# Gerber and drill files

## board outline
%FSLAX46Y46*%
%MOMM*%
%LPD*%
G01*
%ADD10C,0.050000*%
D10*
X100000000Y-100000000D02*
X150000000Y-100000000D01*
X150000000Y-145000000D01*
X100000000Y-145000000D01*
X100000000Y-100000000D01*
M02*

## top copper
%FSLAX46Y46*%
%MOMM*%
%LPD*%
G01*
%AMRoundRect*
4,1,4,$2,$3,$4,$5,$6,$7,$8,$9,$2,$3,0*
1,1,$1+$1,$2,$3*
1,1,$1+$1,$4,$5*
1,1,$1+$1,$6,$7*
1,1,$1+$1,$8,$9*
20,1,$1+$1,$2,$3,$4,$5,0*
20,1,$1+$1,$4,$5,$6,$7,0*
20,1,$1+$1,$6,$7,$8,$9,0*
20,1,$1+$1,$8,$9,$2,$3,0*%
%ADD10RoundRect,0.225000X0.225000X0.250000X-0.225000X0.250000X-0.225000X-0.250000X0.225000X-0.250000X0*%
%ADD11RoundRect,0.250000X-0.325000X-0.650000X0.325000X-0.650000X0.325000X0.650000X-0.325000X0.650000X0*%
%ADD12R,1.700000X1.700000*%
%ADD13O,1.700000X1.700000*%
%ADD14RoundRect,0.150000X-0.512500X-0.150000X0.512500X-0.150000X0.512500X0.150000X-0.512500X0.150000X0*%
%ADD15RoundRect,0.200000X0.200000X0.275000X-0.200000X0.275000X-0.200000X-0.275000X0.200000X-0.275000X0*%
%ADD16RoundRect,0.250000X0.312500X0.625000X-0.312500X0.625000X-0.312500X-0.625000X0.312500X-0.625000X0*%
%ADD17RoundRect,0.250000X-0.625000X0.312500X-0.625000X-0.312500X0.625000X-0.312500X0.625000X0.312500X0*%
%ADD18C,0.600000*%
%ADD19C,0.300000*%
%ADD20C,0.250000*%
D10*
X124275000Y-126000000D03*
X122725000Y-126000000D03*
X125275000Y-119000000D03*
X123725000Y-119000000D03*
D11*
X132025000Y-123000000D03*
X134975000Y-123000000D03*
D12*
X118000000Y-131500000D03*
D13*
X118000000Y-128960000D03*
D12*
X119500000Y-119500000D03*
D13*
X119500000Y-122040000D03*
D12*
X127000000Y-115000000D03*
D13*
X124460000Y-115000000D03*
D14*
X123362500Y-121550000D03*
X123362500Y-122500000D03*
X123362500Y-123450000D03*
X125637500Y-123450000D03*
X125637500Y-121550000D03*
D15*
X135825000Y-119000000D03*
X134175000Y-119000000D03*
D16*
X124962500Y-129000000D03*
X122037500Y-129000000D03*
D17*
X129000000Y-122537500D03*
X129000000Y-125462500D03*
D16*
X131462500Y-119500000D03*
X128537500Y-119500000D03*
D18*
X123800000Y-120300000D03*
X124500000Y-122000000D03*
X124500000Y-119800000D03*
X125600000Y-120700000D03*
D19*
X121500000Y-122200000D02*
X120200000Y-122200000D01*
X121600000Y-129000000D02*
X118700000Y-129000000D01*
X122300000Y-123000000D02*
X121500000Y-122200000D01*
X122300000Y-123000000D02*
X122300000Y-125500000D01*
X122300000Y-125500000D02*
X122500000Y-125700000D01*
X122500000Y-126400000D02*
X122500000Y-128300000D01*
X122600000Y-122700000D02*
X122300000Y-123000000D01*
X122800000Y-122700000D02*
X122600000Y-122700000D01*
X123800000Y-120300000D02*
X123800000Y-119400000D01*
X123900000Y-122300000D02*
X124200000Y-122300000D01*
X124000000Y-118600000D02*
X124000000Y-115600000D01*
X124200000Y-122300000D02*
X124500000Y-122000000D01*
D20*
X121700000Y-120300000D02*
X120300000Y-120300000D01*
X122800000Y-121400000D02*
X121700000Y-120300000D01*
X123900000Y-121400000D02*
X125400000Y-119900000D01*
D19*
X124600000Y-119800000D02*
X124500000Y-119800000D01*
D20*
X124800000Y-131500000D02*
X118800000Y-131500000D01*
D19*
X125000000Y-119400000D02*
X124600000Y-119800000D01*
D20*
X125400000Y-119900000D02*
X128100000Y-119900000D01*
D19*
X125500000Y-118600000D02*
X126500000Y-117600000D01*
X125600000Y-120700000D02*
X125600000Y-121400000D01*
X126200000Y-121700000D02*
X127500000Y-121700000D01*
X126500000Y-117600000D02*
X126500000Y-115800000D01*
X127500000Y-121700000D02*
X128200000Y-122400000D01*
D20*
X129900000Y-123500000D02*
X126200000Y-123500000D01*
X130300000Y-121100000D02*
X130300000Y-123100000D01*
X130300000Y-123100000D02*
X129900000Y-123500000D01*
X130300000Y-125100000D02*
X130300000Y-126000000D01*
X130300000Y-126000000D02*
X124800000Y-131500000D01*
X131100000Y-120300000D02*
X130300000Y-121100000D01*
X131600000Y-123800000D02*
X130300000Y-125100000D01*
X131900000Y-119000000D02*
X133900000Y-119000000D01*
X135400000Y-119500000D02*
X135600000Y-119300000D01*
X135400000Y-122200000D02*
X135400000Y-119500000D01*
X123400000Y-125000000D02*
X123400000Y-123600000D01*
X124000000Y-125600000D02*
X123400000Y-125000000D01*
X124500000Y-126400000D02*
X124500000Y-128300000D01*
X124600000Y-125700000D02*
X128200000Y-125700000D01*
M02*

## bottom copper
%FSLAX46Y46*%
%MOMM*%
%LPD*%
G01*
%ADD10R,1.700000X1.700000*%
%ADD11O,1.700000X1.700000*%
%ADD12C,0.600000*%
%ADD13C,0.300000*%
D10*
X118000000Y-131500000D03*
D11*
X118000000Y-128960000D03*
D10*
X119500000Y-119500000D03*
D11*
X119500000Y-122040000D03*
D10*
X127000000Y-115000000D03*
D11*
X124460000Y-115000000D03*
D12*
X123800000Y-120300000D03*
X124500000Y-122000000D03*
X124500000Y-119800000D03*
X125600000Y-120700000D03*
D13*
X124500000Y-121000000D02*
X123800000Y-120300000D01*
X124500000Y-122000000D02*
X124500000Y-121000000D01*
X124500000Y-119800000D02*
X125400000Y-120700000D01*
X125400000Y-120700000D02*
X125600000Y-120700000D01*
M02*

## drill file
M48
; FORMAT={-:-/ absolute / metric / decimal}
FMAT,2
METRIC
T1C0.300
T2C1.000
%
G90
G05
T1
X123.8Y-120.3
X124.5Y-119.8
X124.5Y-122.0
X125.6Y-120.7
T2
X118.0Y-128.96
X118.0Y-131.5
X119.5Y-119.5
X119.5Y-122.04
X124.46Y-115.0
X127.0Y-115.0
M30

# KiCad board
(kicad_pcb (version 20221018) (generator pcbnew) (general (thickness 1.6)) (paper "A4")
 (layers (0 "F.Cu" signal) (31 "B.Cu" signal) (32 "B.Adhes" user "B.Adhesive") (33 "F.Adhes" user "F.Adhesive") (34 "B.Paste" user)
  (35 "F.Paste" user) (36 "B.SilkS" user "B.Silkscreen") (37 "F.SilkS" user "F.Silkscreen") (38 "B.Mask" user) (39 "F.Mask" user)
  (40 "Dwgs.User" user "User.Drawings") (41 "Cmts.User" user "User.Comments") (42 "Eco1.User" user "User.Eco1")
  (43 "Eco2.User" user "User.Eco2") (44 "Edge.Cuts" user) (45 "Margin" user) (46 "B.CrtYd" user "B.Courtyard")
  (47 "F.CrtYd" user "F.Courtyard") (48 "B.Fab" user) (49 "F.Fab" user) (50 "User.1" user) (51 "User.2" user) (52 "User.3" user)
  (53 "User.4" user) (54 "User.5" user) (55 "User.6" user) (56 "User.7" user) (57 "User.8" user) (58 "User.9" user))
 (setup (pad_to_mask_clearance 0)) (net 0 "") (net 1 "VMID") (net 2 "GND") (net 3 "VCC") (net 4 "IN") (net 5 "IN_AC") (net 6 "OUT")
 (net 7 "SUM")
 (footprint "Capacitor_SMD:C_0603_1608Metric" (layer "F.Cu") (at 123.5 126 180)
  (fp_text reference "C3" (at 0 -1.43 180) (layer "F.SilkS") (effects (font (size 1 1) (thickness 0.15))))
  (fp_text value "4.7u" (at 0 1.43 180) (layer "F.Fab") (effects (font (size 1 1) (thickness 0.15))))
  (pad "1" smd roundrect (at -0.775 0 180) (size 0.9 0.95) (layers "F.Cu" "F.Paste" "F.Mask") (roundrect_rratio 0.25) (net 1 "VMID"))
  (pad "2" smd roundrect (at 0.775 0 180) (size 0.9 0.95) (layers "F.Cu" "F.Paste" "F.Mask") (roundrect_rratio 0.25) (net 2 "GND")))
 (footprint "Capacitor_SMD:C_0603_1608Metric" (layer "F.Cu") (at 124.5 119 180)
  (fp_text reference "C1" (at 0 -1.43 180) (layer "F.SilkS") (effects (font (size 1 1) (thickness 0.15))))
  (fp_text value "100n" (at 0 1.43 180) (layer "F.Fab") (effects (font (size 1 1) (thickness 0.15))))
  (pad "1" smd roundrect (at -0.775 0 180) (size 0.9 0.95) (layers "F.Cu" "F.Paste" "F.Mask") (roundrect_rratio 0.25) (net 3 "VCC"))
  (pad "2" smd roundrect (at 0.775 0 180) (size 0.9 0.95) (layers "F.Cu" "F.Paste" "F.Mask") (roundrect_rratio 0.25) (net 2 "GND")))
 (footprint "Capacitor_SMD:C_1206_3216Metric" (layer "F.Cu") (at 133.5 123)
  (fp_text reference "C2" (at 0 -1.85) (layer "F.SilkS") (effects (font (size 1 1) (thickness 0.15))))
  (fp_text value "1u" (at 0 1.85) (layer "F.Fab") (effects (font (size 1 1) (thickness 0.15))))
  (pad "1" smd roundrect (at -1.475 0) (size 1.15 1.8) (layers "F.Cu" "F.Paste" "F.Mask") (roundrect_rratio 0.217391) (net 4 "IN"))
  (pad "2" smd roundrect (at 1.475 0) (size 1.15 1.8) (layers "F.Cu" "F.Paste" "F.Mask") (roundrect_rratio 0.217391) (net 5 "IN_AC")))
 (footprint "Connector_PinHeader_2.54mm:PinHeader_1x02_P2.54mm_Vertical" (layer "F.Cu") (at 118 131.5 180)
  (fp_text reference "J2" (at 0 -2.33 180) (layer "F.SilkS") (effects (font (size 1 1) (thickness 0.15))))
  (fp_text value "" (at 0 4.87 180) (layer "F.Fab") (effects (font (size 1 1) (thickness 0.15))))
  (pad "1" thru_hole rect (at 0 0 180) (size 1.7 1.7) (drill 1) (layers "*.Cu" "*.Mask") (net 4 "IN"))
  (pad "2" thru_hole oval (at 0 2.54 180) (size 1.7 1.7) (drill 1) (layers "*.Cu" "*.Mask") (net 2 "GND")))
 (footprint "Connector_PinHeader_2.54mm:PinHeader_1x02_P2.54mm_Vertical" (layer "F.Cu") (at 119.5 119.5)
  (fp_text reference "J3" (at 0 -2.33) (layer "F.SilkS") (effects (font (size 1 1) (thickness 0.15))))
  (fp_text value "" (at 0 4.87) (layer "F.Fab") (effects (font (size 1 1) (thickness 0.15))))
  (pad "1" thru_hole rect (at 0 0) (size 1.7 1.7) (drill 1) (layers "*.Cu" "*.Mask") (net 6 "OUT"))
  (pad "2" thru_hole oval (at 0 2.54) (size 1.7 1.7) (drill 1) (layers "*.Cu" "*.Mask") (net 2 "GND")))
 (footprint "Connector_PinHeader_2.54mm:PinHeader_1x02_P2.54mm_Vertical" (layer "F.Cu") (at 127 115 -90)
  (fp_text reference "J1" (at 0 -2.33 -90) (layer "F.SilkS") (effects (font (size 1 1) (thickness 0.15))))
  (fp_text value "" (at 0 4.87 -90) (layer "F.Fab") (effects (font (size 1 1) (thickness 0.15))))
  (pad "1" thru_hole rect (at 0 0 270) (size 1.7 1.7) (drill 1) (layers "*.Cu" "*.Mask") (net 3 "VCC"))
  (pad "2" thru_hole oval (at 0 2.54 270) (size 1.7 1.7) (drill 1) (layers "*.Cu" "*.Mask") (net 2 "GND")))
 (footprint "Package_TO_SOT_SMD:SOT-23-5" (layer "F.Cu") (at 124.5 122.5)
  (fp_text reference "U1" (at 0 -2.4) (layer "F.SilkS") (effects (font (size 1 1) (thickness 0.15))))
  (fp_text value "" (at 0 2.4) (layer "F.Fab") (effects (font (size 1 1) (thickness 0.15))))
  (pad "1" smd roundrect (at -1.1375 -0.95) (size 1.325 0.6) (layers "F.Cu" "F.Paste" "F.Mask") (roundrect_rratio 0.25) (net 6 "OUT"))
  (pad "2" smd roundrect (at -1.1375 0) (size 1.325 0.6) (layers "F.Cu" "F.Paste" "F.Mask") (roundrect_rratio 0.25) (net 2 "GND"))
  (pad "3" smd roundrect (at -1.1375 0.95) (size 1.325 0.6) (layers "F.Cu" "F.Paste" "F.Mask") (roundrect_rratio 0.25) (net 1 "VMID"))
  (pad "4" smd roundrect (at 1.1375 0.95) (size 1.325 0.6) (layers "F.Cu" "F.Paste" "F.Mask") (roundrect_rratio 0.25) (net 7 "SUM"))
  (pad "5" smd roundrect (at 1.1375 -0.95) (size 1.325 0.6) (layers "F.Cu" "F.Paste" "F.Mask") (roundrect_rratio 0.25) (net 3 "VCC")))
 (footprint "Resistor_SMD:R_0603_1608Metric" (layer "F.Cu") (at 135 119 180)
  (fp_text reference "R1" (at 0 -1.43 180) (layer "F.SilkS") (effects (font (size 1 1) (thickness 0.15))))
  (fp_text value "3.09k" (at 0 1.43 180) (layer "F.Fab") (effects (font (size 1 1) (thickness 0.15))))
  (pad "1" smd roundrect (at -0.825 0 180) (size 0.8 0.95) (layers "F.Cu" "F.Paste" "F.Mask") (roundrect_rratio 0.25) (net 5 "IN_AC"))
  (pad "2" smd roundrect (at 0.825 0 180) (size 0.8 0.95) (layers "F.Cu" "F.Paste" "F.Mask") (roundrect_rratio 0.25) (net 7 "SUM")))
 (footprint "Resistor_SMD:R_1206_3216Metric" (layer "F.Cu") (at 123.5 129 180)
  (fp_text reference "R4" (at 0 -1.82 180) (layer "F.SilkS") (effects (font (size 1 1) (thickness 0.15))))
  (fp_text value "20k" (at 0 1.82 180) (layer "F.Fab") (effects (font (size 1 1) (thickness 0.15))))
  (pad "1" smd roundrect (at -1.4625 0 180) (size 1.125 1.75) (layers "F.Cu" "F.Paste" "F.Mask") (roundrect_rratio 0.222222) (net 1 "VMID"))
  (pad "2" smd roundrect (at 1.4625 0 180) (size 1.125 1.75) (layers "F.Cu" "F.Paste" "F.Mask") (roundrect_rratio 0.222222) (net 2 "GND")))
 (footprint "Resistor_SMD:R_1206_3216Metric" (layer "F.Cu") (at 129 124 -90)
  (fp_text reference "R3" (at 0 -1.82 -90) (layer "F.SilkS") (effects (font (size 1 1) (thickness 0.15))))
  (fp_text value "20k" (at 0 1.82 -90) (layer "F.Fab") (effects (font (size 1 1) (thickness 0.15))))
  (pad "1" smd roundrect (at -1.4625 0 270) (size 1.125 1.75) (layers "F.Cu" "F.Paste" "F.Mask") (roundrect_rratio 0.222222) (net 3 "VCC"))
  (pad "2" smd roundrect (at 1.4625 0 270) (size 1.125 1.75) (layers "F.Cu" "F.Paste" "F.Mask") (roundrect_rratio 0.222222) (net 1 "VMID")))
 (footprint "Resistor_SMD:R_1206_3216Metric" (layer "F.Cu") (at 130 119.5 180)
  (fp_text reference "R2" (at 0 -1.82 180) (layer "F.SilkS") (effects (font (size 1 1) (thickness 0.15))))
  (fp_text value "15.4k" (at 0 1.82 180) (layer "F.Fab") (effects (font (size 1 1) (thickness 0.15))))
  (pad "1" smd roundrect (at -1.4625 0 180) (size 1.125 1.75) (layers "F.Cu" "F.Paste" "F.Mask") (roundrect_rratio 0.222222) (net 7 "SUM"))
  (pad "2" smd roundrect (at 1.4625 0 180) (size 1.125 1.75) (layers "F.Cu" "F.Paste" "F.Mask") (roundrect_rratio 0.222222) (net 6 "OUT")))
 (gr_rect (start 100 100) (end 150 145) (stroke (width 0.05) (type default)) (fill none) (layer "Edge.Cuts"))
 (segment (start 121.5 122.2) (end 120.2 122.2) (width 0.3) (layer "F.Cu") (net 2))
 (segment (start 121.6 129) (end 118.7 129) (width 0.3) (layer "F.Cu") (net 2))
 (segment (start 122.3 123) (end 121.5 122.2) (width 0.3) (layer "F.Cu") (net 2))
 (segment (start 122.3 123) (end 122.3 125.5) (width 0.3) (layer "F.Cu") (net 2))
 (segment (start 122.3 125.5) (end 122.5 125.7) (width 0.3) (layer "F.Cu") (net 2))
 (segment (start 122.5 126.4) (end 122.5 128.3) (width 0.3) (layer "F.Cu") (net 2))
 (segment (start 122.6 122.7) (end 122.3 123) (width 0.3) (layer "F.Cu") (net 2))
 (segment (start 122.8 122.7) (end 122.6 122.7) (width 0.3) (layer "F.Cu") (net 2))
 (segment (start 123.8 120.3) (end 123.8 119.4) (width 0.3) (layer "F.Cu") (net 2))
 (segment (start 123.9 122.3) (end 124.2 122.3) (width 0.3) (layer "F.Cu") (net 2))
 (segment (start 124 118.6) (end 124 115.6) (width 0.3) (layer "F.Cu") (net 2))
 (segment (start 124.2 122.3) (end 124.5 122) (width 0.3) (layer "F.Cu") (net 2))
 (via (at 123.8 120.3) (size 0.6) (drill 0.3) (layers "F.Cu" "B.Cu") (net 2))
 (via (at 124.5 122) (size 0.6) (drill 0.3) (layers "F.Cu" "B.Cu") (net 2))
 (segment (start 121.7 120.3) (end 120.3 120.3) (width 0.25) (layer "F.Cu") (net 6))
 (segment (start 122.8 121.4) (end 121.7 120.3) (width 0.25) (layer "F.Cu") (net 6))
 (segment (start 123.9 121.4) (end 125.4 119.9) (width 0.25) (layer "F.Cu") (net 6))
 (segment (start 124.5 121) (end 123.8 120.3) (width 0.3) (layer "B.Cu") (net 2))
 (segment (start 124.5 122) (end 124.5 121) (width 0.3) (layer "B.Cu") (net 2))
 (segment (start 124.6 119.8) (end 124.5 119.8) (width 0.3) (layer "F.Cu") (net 3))
 (segment (start 124.8 131.5) (end 118.8 131.5) (width 0.25) (layer "F.Cu") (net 4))
 (segment (start 125 119.4) (end 124.6 119.8) (width 0.3) (layer "F.Cu") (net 3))
 (segment (start 125.4 119.9) (end 128.1 119.9) (width 0.25) (layer "F.Cu") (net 6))
 (segment (start 125.5 118.6) (end 126.5 117.6) (width 0.3) (layer "F.Cu") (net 3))
 (segment (start 125.6 120.7) (end 125.6 121.4) (width 0.3) (layer "F.Cu") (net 3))
 (segment (start 126.2 121.7) (end 127.5 121.7) (width 0.3) (layer "F.Cu") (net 3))
 (segment (start 126.5 117.6) (end 126.5 115.8) (width 0.3) (layer "F.Cu") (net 3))
 (segment (start 127.5 121.7) (end 128.2 122.4) (width 0.3) (layer "F.Cu") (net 3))
 (segment (start 129.9 123.5) (end 126.2 123.5) (width 0.25) (layer "F.Cu") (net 7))
 (segment (start 130.3 121.1) (end 130.3 123.1) (width 0.25) (layer "F.Cu") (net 7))
 (segment (start 130.3 123.1) (end 129.9 123.5) (width 0.25) (layer "F.Cu") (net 7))
 (segment (start 130.3 125.1) (end 130.3 126) (width 0.25) (layer "F.Cu") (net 4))
 (segment (start 130.3 126) (end 124.8 131.5) (width 0.25) (layer "F.Cu") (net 4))
 (segment (start 131.1 120.3) (end 130.3 121.1) (width 0.25) (layer "F.Cu") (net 7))
 (segment (start 131.6 123.8) (end 130.3 125.1) (width 0.25) (layer "F.Cu") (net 4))
 (segment (start 131.9 119) (end 133.9 119) (width 0.25) (layer "F.Cu") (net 7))
 (segment (start 135.4 119.5) (end 135.6 119.3) (width 0.25) (layer "F.Cu") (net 5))
 (segment (start 135.4 122.2) (end 135.4 119.5) (width 0.25) (layer "F.Cu") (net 5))
 (via (at 124.5 119.8) (size 0.6) (drill 0.3) (layers "F.Cu" "B.Cu") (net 3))
 (via (at 125.6 120.7) (size 0.6) (drill 0.3) (layers "F.Cu" "B.Cu") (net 3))
 (segment (start 123.4 125) (end 123.4 123.6) (width 0.25) (layer "F.Cu") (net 1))
 (segment (start 124 125.6) (end 123.4 125) (width 0.25) (layer "F.Cu") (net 1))
 (segment (start 124.5 119.8) (end 125.4 120.7) (width 0.3) (layer "B.Cu") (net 3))
 (segment (start 124.5 126.4) (end 124.5 128.3) (width 0.25) (layer "F.Cu") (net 1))
 (segment (start 124.6 125.7) (end 128.2 125.7) (width 0.25) (layer "F.Cu") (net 1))
 (segment (start 125.4 120.7) (end 125.6 120.7) (width 0.3) (layer "B.Cu") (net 3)))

